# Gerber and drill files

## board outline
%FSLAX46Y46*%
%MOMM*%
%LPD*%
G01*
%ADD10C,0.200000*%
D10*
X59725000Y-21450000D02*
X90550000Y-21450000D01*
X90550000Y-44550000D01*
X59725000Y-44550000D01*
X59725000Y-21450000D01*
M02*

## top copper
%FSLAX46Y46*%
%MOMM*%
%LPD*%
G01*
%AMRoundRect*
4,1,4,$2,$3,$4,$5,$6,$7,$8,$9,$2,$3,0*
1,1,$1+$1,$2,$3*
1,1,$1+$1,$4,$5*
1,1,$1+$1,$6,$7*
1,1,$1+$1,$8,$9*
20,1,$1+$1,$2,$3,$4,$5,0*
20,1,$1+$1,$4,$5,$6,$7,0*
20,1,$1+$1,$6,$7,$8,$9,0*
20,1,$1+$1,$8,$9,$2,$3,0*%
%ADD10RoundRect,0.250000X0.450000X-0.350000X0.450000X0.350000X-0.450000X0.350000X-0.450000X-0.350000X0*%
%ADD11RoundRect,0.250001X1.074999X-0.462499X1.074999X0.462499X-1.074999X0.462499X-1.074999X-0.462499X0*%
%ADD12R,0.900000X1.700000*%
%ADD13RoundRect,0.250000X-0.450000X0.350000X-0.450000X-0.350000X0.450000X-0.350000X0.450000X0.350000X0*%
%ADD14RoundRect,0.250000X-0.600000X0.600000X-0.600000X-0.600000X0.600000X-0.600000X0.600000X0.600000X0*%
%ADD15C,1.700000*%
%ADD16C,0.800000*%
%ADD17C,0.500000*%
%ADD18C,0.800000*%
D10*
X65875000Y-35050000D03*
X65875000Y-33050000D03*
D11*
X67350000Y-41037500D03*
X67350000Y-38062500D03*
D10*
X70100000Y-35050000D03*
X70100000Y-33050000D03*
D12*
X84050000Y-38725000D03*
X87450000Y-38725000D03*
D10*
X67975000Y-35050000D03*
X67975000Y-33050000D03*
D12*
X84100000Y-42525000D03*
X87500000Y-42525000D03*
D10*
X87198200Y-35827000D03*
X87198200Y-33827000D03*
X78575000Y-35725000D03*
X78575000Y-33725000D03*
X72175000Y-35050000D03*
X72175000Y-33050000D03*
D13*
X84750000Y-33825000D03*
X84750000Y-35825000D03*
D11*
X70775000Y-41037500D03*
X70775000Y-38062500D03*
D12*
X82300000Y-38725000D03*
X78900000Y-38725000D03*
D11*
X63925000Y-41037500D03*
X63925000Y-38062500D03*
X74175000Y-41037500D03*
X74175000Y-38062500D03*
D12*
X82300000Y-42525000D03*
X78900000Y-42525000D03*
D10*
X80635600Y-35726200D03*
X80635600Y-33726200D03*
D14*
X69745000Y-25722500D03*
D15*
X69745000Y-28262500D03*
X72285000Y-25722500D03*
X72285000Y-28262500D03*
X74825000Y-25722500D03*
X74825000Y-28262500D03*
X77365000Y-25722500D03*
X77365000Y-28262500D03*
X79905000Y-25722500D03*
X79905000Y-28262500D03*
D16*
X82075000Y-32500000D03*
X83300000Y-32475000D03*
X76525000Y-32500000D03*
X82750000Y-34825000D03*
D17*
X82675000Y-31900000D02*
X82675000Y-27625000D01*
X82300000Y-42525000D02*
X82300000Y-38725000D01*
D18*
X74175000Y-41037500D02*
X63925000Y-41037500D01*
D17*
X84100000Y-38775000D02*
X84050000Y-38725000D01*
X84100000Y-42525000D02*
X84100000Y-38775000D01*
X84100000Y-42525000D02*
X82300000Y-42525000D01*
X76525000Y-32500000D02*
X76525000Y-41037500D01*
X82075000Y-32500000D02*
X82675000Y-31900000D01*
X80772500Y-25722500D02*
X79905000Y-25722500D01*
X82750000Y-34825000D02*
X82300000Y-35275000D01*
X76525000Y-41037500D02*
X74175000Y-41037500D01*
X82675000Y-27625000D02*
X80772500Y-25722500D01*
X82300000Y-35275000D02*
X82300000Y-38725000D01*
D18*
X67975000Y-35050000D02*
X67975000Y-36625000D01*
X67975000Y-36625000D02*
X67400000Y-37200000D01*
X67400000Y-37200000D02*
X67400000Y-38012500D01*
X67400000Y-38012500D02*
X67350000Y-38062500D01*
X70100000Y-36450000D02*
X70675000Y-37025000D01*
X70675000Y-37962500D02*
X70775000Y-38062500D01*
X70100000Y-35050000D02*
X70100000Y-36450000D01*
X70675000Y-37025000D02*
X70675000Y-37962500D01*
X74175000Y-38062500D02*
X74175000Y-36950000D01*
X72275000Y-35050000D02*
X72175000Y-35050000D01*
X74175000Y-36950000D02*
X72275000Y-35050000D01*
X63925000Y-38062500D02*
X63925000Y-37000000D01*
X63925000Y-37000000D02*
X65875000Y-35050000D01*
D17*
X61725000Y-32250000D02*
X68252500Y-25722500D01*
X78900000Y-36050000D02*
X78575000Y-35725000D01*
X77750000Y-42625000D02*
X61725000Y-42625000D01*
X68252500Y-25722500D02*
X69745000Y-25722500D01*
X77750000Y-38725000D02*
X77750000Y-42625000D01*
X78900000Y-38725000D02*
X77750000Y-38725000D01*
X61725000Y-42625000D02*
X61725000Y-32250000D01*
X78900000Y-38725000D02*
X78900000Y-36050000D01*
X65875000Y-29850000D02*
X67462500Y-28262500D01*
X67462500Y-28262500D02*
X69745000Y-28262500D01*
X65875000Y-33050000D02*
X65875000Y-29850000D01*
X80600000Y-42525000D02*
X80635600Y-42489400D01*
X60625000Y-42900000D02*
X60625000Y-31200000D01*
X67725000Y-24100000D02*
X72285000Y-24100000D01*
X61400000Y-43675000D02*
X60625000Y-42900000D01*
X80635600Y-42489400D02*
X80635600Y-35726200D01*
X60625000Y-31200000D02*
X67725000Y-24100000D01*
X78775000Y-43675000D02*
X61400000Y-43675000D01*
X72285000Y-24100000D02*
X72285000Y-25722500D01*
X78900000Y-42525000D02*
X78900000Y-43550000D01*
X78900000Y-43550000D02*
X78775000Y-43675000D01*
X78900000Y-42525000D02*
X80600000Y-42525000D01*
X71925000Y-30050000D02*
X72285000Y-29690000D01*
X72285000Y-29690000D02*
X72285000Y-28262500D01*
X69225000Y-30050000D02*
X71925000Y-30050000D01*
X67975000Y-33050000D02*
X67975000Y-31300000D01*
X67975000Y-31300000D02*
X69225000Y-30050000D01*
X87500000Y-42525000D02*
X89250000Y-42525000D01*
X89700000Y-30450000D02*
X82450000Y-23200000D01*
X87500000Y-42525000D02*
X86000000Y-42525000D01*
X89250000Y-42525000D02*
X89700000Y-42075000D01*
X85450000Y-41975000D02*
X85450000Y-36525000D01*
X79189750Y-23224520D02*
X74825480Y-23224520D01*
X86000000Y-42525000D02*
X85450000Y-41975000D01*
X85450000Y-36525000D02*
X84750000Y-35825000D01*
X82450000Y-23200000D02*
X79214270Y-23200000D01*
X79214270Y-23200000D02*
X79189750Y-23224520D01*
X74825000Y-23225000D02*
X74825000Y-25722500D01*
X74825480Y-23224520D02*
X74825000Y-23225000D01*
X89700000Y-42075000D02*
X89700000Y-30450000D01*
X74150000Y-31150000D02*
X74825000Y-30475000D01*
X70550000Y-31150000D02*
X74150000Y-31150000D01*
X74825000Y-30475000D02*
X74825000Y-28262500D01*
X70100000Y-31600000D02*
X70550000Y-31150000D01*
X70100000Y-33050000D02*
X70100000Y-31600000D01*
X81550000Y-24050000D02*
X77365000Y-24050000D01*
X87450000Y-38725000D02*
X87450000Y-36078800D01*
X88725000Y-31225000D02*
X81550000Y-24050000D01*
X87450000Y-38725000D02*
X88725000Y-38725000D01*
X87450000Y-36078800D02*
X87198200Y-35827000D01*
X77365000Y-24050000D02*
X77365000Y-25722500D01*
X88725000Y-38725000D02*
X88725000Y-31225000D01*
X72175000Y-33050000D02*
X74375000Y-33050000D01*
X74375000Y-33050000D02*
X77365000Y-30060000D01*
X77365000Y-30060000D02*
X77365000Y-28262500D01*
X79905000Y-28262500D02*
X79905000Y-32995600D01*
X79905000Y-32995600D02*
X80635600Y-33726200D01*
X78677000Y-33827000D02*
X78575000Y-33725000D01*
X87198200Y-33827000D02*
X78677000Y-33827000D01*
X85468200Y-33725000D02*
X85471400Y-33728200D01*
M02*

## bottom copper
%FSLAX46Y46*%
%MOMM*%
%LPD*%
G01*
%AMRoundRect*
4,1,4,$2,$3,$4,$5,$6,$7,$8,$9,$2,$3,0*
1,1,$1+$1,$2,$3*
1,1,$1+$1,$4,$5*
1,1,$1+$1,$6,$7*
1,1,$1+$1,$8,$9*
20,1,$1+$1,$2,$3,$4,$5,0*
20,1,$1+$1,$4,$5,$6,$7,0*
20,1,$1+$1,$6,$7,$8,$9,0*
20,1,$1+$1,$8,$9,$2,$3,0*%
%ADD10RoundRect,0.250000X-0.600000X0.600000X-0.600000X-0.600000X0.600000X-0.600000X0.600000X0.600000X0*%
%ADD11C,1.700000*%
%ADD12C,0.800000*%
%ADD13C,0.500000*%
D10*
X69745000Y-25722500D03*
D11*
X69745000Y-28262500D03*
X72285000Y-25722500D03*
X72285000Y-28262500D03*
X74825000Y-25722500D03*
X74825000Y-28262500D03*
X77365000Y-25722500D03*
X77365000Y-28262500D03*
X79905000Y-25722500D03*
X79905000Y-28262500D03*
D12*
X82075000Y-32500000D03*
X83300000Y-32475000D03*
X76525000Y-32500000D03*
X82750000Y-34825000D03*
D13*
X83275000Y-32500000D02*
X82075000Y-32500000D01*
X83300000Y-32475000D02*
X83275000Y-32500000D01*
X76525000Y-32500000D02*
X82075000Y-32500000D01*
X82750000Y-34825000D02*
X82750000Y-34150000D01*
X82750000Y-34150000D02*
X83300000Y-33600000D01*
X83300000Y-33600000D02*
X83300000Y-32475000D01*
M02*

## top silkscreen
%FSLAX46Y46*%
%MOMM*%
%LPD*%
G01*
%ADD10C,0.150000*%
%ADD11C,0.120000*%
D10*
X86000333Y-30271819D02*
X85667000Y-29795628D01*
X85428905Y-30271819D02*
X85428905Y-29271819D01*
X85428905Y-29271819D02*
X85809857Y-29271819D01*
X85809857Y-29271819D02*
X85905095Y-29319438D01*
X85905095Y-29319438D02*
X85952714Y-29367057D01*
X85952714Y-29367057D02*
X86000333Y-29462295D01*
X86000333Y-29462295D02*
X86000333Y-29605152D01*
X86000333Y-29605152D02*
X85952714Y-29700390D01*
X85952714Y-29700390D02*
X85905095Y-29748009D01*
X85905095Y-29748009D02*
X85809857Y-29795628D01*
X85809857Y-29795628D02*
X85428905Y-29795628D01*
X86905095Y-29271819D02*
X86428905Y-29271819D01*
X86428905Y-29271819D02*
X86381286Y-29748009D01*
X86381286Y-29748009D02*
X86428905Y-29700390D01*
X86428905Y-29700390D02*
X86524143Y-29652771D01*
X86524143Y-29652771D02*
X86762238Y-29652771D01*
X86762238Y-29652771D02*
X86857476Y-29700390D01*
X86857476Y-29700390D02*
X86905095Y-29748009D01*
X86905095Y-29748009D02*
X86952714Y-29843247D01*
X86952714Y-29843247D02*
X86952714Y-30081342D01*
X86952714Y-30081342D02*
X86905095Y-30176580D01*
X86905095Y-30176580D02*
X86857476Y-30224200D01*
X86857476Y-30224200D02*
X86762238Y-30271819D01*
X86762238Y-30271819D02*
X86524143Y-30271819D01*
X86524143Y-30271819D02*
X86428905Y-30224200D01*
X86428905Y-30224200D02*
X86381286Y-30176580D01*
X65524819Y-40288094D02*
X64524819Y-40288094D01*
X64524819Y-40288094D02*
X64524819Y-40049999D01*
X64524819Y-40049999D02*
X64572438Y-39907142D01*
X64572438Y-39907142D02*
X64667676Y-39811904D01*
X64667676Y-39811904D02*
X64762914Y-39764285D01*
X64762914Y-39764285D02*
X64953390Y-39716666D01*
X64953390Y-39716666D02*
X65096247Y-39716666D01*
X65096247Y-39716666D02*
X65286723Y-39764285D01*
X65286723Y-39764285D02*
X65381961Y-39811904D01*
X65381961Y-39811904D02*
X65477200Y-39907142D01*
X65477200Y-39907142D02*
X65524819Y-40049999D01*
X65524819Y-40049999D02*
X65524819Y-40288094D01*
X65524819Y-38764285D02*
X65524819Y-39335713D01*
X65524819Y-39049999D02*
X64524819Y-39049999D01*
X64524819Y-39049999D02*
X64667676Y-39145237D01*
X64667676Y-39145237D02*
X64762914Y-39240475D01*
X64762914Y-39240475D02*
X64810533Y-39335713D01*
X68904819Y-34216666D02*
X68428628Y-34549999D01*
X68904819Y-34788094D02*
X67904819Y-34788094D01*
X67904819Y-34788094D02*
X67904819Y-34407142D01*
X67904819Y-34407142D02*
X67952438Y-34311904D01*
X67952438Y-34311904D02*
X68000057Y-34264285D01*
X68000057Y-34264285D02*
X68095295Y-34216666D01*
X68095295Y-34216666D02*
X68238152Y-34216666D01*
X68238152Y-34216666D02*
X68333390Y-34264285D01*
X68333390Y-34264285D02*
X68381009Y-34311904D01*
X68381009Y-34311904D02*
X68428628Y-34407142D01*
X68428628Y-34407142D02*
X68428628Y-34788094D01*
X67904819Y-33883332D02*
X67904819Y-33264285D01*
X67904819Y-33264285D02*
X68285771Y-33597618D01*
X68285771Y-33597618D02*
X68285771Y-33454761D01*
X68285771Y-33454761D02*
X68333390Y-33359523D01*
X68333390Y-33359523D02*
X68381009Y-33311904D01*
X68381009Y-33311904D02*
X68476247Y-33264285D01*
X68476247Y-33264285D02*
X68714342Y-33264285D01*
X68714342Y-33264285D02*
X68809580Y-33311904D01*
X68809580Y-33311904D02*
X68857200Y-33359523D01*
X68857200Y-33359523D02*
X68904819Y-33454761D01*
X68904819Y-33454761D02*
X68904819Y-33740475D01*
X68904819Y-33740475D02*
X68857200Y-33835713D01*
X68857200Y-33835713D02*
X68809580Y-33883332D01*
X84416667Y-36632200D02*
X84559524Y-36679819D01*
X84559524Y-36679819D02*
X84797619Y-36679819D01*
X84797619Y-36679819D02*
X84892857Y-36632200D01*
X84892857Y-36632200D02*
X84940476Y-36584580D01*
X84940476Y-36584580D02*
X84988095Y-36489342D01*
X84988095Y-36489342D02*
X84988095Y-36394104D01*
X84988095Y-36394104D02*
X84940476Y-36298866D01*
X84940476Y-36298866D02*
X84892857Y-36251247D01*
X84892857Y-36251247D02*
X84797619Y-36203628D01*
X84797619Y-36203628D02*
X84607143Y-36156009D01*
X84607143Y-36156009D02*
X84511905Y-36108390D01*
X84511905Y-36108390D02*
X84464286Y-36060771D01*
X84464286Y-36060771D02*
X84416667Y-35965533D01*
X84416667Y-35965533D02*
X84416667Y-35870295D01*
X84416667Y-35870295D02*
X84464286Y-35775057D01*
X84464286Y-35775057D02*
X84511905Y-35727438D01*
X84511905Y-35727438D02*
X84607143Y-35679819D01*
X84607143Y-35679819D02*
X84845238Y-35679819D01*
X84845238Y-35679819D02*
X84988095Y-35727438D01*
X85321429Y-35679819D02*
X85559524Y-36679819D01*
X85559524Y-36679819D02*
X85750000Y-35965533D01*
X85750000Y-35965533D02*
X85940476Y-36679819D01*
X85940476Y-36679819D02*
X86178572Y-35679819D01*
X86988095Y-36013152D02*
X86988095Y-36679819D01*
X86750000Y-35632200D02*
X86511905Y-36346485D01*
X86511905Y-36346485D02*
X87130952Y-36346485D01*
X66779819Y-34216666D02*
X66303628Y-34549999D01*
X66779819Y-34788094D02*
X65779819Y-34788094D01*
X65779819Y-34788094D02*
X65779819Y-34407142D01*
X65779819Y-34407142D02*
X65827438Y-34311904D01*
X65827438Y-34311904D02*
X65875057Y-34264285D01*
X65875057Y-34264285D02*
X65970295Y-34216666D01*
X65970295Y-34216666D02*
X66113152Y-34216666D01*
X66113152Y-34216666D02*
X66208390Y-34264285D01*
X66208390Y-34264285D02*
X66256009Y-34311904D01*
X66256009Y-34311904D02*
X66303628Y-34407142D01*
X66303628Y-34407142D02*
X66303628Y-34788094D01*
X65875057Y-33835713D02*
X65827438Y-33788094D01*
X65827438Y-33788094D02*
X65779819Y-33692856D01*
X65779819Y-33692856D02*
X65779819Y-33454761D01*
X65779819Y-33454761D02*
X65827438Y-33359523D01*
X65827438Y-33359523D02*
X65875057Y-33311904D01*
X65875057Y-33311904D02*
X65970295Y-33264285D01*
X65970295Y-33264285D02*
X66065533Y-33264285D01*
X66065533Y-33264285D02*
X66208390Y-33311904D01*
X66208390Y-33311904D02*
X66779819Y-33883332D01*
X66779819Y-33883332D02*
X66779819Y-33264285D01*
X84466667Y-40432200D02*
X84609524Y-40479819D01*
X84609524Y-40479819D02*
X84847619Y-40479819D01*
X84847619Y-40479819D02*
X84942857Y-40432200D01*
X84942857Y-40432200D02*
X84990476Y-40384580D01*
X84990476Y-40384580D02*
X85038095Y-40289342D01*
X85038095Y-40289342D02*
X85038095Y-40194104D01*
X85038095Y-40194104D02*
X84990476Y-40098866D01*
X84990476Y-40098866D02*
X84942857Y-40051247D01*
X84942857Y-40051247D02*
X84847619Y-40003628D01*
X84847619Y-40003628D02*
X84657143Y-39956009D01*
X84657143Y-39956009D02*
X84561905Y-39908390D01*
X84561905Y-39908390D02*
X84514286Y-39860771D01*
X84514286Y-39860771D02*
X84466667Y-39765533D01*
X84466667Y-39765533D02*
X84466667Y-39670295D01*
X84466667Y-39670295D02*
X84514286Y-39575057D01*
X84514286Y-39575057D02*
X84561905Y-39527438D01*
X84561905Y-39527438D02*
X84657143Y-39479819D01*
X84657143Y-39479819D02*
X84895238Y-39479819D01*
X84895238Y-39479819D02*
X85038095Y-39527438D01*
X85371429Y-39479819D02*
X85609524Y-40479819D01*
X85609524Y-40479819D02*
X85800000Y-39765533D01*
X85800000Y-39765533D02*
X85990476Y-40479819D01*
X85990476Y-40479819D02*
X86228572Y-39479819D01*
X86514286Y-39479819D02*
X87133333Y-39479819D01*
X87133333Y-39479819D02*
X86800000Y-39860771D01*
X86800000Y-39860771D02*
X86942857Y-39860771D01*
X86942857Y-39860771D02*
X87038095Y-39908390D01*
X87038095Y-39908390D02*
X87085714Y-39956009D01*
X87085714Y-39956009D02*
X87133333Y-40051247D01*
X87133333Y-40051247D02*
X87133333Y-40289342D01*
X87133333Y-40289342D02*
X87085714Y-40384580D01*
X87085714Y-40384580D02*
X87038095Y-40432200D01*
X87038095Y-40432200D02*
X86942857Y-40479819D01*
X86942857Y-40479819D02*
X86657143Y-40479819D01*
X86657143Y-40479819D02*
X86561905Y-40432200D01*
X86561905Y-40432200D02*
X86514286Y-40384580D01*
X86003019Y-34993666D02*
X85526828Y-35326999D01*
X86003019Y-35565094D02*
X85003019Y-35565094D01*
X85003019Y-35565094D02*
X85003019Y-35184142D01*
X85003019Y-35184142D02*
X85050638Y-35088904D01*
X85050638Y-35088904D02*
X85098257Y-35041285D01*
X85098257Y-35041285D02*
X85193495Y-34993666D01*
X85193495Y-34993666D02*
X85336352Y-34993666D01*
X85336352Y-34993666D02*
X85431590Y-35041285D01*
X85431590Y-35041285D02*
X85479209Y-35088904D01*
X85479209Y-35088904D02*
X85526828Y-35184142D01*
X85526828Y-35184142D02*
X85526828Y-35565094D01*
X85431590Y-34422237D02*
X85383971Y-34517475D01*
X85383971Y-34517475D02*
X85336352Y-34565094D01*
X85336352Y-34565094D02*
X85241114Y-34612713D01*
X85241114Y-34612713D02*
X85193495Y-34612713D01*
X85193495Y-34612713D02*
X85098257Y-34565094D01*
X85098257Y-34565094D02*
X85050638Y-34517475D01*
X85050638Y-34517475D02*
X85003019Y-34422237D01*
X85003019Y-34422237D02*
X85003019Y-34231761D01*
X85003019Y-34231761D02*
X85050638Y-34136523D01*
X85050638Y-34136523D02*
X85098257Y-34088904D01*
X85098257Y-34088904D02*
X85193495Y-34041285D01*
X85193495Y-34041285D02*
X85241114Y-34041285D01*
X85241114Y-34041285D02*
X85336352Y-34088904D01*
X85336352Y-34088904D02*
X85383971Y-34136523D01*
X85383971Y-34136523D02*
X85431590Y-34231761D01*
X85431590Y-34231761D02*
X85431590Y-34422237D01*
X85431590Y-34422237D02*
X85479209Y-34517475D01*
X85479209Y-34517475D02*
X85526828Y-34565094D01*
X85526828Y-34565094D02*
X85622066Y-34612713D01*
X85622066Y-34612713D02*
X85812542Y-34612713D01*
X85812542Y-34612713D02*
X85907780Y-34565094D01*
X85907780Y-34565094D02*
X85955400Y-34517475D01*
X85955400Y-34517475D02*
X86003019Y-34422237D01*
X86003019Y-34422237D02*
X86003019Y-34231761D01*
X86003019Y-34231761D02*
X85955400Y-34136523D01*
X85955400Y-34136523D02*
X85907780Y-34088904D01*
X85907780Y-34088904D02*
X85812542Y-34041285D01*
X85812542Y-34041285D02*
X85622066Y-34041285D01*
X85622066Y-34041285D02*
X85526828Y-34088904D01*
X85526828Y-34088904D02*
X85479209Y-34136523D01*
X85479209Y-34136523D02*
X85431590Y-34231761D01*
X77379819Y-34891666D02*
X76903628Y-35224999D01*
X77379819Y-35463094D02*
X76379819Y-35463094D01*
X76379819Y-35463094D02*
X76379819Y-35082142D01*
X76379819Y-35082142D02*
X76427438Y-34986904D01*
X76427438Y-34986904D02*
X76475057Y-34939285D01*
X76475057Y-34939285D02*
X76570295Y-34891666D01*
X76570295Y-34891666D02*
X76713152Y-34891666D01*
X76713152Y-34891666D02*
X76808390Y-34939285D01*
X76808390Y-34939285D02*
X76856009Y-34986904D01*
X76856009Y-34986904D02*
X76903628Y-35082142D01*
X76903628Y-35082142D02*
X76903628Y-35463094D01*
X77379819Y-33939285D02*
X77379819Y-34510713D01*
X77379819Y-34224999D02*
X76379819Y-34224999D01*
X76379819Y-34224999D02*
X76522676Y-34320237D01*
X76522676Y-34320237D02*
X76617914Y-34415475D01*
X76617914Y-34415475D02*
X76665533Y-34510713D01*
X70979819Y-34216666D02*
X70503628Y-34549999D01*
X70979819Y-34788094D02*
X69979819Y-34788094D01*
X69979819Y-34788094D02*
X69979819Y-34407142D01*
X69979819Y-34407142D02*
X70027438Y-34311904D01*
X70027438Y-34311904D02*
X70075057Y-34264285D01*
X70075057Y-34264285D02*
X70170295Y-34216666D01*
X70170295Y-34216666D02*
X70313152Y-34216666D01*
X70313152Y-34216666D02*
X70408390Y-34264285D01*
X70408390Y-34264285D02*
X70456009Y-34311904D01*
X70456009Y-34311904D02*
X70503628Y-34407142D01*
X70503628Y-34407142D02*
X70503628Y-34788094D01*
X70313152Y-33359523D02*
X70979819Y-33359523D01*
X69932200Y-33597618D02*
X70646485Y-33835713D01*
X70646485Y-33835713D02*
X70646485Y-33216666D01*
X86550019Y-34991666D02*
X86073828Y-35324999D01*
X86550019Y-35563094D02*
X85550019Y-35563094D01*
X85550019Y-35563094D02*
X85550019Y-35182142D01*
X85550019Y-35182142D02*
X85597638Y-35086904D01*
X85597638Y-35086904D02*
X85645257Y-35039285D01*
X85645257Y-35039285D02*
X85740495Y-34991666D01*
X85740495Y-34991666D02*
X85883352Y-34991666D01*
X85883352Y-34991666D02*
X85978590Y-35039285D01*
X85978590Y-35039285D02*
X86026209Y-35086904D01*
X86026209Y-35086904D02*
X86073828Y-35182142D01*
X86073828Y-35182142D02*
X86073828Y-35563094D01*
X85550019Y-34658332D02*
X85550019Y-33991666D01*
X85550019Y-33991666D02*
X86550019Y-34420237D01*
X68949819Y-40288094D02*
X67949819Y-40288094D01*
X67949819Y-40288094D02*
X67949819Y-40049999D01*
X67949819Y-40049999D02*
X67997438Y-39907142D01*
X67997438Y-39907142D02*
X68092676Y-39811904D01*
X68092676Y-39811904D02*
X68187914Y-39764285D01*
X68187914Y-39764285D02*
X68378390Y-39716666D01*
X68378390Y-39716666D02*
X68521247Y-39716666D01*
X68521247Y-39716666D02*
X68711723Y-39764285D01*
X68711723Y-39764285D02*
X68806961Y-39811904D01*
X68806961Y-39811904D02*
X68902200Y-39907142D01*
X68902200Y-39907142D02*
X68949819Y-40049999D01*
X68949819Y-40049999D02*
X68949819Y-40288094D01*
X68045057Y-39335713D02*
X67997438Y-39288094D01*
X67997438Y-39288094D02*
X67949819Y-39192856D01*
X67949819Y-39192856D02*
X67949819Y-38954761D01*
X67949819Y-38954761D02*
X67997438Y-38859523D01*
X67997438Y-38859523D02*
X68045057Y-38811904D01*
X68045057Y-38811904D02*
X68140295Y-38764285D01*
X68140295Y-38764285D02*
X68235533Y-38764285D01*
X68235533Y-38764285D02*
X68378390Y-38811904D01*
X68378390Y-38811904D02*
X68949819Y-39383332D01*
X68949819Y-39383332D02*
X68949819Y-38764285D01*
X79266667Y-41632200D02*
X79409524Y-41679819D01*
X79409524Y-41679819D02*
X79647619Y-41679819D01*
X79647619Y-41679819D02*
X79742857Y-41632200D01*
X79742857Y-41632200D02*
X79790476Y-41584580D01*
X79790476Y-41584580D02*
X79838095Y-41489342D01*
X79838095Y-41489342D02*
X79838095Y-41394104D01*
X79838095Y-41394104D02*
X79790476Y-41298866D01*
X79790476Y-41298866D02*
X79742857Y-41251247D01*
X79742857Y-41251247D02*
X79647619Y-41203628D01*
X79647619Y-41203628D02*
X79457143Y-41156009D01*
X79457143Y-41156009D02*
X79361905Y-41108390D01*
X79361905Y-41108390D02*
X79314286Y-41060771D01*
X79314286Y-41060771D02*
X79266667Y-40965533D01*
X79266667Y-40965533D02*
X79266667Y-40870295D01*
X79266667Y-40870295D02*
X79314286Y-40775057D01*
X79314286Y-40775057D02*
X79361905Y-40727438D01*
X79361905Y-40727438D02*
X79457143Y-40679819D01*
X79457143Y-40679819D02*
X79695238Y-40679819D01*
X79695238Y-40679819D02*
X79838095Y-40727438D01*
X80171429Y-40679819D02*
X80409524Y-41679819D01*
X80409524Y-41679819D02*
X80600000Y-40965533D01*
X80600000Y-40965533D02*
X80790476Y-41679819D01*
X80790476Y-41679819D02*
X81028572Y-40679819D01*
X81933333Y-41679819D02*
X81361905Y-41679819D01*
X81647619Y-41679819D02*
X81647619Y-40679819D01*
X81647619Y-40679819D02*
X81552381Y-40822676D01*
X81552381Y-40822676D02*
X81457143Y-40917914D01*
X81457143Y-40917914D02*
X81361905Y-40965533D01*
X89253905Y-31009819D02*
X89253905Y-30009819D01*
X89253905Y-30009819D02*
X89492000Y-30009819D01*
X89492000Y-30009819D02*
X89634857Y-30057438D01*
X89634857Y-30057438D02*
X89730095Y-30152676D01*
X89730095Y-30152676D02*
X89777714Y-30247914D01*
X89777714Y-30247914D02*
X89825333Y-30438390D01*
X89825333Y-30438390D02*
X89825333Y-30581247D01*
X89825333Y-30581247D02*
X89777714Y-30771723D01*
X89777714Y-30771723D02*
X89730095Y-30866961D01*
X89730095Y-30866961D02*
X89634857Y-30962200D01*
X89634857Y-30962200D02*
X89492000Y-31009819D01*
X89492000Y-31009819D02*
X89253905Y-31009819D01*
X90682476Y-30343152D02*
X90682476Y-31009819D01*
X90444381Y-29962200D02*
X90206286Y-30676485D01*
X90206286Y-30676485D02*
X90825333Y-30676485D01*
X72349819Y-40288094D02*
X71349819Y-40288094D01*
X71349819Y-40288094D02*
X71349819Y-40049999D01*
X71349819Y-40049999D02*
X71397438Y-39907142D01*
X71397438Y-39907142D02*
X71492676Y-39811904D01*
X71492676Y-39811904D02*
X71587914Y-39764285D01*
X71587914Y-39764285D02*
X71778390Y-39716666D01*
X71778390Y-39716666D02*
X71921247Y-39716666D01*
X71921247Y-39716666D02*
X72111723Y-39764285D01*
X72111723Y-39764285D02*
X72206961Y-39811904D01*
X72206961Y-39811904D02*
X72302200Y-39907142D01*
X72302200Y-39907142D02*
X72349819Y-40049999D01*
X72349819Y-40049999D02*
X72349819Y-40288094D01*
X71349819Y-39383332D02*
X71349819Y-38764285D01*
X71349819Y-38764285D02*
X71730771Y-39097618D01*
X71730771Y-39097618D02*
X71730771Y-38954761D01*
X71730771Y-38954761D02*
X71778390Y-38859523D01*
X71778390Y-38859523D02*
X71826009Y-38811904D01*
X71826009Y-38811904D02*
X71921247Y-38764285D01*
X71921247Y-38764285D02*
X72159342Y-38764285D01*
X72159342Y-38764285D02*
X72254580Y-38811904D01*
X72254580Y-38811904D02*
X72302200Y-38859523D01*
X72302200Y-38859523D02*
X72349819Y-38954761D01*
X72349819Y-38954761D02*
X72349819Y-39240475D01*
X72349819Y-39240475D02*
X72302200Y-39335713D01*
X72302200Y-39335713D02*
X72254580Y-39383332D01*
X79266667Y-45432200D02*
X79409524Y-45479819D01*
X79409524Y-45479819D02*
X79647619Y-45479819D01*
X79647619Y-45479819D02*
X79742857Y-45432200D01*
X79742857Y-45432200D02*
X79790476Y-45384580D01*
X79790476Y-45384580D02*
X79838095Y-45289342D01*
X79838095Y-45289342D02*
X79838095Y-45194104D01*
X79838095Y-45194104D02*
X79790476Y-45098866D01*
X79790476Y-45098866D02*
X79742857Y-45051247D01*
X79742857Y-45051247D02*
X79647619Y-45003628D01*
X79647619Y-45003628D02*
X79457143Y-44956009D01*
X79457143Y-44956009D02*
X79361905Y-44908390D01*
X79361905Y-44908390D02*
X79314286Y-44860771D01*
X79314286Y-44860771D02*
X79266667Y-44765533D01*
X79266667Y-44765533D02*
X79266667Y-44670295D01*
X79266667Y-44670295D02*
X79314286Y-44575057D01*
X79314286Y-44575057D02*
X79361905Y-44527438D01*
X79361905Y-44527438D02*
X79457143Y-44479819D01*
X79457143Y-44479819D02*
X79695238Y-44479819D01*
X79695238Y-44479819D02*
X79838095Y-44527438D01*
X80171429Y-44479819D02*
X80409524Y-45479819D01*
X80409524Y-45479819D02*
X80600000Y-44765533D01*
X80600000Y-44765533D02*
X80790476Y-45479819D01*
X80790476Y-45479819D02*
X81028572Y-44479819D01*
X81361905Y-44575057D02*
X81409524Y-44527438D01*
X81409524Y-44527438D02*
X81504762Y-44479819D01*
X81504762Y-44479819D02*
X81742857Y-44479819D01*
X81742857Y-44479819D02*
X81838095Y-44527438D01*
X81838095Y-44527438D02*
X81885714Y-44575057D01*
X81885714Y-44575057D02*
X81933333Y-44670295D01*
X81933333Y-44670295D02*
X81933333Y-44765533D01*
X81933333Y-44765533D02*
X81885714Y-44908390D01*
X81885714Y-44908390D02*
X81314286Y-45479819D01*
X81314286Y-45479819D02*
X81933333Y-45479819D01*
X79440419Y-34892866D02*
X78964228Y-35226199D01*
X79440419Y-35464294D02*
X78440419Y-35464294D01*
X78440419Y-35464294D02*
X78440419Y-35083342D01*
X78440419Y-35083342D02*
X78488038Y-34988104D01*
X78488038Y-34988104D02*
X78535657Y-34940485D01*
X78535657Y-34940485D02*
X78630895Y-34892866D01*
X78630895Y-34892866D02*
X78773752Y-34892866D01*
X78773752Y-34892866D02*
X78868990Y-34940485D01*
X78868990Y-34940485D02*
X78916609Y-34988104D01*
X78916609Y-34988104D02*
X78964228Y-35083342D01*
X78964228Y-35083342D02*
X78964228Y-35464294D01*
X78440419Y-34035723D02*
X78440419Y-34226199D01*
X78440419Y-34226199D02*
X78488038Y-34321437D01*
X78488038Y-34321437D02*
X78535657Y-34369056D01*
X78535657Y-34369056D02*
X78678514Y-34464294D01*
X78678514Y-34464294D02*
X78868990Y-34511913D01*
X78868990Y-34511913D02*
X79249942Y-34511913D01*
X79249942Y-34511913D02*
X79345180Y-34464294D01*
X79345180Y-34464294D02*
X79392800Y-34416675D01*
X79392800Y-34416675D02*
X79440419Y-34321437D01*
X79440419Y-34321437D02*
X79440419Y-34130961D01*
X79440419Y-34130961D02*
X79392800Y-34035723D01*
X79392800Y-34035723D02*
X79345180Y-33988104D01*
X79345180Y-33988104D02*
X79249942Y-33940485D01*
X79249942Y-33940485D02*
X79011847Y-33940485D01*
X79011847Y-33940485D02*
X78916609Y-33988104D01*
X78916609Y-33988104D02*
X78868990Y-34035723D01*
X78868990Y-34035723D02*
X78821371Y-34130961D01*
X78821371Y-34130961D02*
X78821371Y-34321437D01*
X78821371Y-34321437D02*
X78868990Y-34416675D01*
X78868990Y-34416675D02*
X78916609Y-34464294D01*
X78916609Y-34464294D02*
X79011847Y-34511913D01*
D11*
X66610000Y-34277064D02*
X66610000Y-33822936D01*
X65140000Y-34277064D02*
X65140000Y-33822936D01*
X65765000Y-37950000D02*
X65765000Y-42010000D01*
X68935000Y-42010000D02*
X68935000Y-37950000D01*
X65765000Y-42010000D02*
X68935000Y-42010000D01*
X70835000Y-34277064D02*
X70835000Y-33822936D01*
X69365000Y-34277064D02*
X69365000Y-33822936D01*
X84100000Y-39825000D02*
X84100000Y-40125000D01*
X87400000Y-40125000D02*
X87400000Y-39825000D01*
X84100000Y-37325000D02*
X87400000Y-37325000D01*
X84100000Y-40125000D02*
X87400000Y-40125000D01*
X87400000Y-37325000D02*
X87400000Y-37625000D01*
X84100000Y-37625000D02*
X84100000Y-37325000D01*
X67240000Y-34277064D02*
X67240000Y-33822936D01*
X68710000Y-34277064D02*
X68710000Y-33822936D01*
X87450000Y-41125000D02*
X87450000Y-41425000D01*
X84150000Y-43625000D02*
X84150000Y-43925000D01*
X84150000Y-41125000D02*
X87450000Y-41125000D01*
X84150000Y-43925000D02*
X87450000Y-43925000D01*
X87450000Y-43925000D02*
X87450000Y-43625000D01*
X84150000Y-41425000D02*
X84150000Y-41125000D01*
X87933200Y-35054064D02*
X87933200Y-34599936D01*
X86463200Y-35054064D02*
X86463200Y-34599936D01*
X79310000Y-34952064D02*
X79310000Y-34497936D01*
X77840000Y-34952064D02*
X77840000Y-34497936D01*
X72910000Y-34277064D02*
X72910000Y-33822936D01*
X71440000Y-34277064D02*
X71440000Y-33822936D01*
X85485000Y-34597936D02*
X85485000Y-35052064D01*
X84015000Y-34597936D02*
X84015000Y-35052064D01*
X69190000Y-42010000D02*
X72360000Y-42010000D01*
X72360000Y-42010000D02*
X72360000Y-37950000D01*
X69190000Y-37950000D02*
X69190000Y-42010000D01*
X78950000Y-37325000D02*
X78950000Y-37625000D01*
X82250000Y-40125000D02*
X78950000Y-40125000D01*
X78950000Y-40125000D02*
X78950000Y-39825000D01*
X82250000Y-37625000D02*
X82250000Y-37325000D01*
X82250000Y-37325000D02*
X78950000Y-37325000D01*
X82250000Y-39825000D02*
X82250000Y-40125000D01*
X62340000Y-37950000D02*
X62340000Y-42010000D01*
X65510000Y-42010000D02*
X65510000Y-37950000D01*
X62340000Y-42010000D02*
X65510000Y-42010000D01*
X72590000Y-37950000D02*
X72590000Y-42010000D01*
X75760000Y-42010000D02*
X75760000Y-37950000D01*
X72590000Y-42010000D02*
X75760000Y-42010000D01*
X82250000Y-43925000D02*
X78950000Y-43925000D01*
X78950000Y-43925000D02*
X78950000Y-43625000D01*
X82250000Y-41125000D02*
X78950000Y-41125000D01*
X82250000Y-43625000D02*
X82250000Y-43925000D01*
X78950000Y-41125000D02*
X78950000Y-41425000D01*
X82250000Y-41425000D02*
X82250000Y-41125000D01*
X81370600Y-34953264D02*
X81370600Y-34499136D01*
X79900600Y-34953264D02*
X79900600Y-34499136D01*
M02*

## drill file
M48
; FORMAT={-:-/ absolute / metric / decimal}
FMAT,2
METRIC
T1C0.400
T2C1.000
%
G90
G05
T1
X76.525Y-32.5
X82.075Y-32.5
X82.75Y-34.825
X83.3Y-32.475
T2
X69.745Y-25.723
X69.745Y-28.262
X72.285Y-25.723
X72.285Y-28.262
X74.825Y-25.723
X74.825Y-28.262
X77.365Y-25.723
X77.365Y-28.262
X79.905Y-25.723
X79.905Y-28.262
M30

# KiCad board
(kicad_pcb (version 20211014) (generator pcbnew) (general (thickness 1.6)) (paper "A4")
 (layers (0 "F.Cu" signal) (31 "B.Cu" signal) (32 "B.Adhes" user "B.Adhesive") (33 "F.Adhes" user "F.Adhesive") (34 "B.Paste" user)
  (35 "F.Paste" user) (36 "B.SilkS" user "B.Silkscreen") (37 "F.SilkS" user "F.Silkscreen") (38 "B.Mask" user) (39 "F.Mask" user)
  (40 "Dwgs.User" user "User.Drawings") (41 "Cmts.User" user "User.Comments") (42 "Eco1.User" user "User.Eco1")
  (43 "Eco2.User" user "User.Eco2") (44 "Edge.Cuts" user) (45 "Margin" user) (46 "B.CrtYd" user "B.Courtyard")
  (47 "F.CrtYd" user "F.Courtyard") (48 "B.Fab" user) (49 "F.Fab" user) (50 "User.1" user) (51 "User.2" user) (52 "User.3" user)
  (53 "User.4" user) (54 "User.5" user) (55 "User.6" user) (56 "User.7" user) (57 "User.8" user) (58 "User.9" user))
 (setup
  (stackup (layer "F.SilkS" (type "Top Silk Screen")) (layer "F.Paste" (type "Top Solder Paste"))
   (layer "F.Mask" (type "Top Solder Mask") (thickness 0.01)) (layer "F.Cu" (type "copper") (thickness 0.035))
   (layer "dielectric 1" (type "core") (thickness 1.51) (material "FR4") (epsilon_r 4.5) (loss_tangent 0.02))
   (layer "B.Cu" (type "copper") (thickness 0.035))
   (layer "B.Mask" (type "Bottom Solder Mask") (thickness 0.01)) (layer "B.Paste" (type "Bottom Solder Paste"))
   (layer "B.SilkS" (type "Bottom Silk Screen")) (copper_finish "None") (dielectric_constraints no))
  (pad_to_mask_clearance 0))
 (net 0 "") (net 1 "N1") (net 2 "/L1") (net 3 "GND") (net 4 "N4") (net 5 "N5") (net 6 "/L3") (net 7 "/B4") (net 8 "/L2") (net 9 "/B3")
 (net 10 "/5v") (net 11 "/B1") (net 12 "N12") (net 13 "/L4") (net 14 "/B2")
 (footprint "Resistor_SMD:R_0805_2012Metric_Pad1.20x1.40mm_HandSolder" (layer "F.Cu") (at 65.875 34.05 90)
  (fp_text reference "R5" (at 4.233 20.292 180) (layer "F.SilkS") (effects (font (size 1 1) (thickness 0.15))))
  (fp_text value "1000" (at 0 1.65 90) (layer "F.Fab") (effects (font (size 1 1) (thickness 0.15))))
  (fp_line (start -0.227064 0.735) (end 0.227064 0.735) (layer "F.SilkS") (width 0.12))
  (fp_line (start -0.227064 -0.735) (end 0.227064 -0.735) (layer "F.SilkS") (width 0.12))
  (pad "1" smd roundrect (at -1 0 90) (size 1.2 1.4) (layers "F.Cu" "F.Paste" "F.Mask") (roundrect_rratio 0.208333) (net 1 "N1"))
  (pad "2" smd roundrect (at 1 0 90) (size 1.2 1.4) (layers "F.Cu" "F.Paste" "F.Mask") (roundrect_rratio 0.208333) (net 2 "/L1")))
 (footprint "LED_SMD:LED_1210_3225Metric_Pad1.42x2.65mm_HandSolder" (layer "F.Cu") (at 67.35 39.55 90)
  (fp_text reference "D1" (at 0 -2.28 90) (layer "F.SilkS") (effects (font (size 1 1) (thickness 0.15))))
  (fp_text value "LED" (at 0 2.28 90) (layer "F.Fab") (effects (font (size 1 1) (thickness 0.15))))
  (fp_line (start 1.6 -1.585) (end -2.46 -1.585) (layer "F.SilkS") (width 0.12))
  (fp_line (start -2.46 1.585) (end 1.6 1.585) (layer "F.SilkS") (width 0.12))
  (fp_line (start -2.46 -1.585) (end -2.46 1.585) (layer "F.SilkS") (width 0.12))
  (pad "1" smd roundrect (at -1.4875 0 90) (size 1.425 2.65) (layers "F.Cu" "F.Paste" "F.Mask") (roundrect_rratio 0.175439) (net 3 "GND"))
  (pad "2" smd roundrect (at 1.4875 0 90) (size 1.425 2.65) (layers "F.Cu" "F.Paste" "F.Mask") (roundrect_rratio 0.175439) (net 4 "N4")))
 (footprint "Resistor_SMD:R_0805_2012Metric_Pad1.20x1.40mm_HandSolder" (layer "F.Cu") (at 70.1 34.05 90)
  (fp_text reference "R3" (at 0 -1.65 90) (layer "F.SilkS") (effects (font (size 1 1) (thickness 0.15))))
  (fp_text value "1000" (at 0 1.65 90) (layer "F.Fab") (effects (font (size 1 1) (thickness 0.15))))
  (fp_line (start -0.227064 0.735) (end 0.227064 0.735) (layer "F.SilkS") (width 0.12))
  (fp_line (start -0.227064 -0.735) (end 0.227064 -0.735) (layer "F.SilkS") (width 0.12))
  (pad "1" smd roundrect (at -1 0 90) (size 1.2 1.4) (layers "F.Cu" "F.Paste" "F.Mask") (roundrect_rratio 0.208333) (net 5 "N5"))
  (pad "2" smd roundrect (at 1 0 90) (size 1.2 1.4) (layers "F.Cu" "F.Paste" "F.Mask") (roundrect_rratio 0.208333) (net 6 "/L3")))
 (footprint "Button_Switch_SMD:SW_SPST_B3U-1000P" (layer "F.Cu") (at 85.75 38.725)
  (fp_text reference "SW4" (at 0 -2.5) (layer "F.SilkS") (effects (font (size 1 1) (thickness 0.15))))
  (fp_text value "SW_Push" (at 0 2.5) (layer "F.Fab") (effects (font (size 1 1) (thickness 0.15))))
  (fp_line (start -1.65 1.1) (end -1.65 1.4) (layer "F.SilkS") (width 0.12))
  (fp_line (start 1.65 1.4) (end 1.65 1.1) (layer "F.SilkS") (width 0.12))
  (fp_line (start -1.65 -1.4) (end 1.65 -1.4) (layer "F.SilkS") (width 0.12))
  (fp_line (start -1.65 1.4) (end 1.65 1.4) (layer "F.SilkS") (width 0.12))
  (fp_line (start 1.65 -1.4) (end 1.65 -1.1) (layer "F.SilkS") (width 0.12))
  (fp_line (start -1.65 -1.1) (end -1.65 -1.4) (layer "F.SilkS") (width 0.12))
  (pad "1" smd rect (at -1.7 0) (size 0.9 1.7) (layers "F.Cu" "F.Paste" "F.Mask") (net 3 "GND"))
  (pad "2" smd rect (at 1.7 0) (size 0.9 1.7) (layers "F.Cu" "F.Paste" "F.Mask") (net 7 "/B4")))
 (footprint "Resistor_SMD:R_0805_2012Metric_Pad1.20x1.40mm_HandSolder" (layer "F.Cu") (at 67.975 34.05 90)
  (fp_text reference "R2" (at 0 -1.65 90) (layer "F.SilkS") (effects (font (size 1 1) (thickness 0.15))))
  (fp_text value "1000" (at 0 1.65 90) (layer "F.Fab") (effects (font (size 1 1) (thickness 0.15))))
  (fp_line (start -0.227064 -0.735) (end 0.227064 -0.735) (layer "F.SilkS") (width 0.12))
  (fp_line (start -0.227064 0.735) (end 0.227064 0.735) (layer "F.SilkS") (width 0.12))
  (pad "1" smd roundrect (at -1 0 90) (size 1.2 1.4) (layers "F.Cu" "F.Paste" "F.Mask") (roundrect_rratio 0.208333) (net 4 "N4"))
  (pad "2" smd roundrect (at 1 0 90) (size 1.2 1.4) (layers "F.Cu" "F.Paste" "F.Mask") (roundrect_rratio 0.208333) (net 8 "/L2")))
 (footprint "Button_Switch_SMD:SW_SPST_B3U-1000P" (layer "F.Cu") (at 85.8 42.525)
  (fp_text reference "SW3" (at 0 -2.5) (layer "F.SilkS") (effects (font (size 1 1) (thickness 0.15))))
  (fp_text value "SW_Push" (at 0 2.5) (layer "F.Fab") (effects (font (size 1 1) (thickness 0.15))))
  (fp_line (start 1.65 -1.4) (end 1.65 -1.1) (layer "F.SilkS") (width 0.12))
  (fp_line (start -1.65 1.1) (end -1.65 1.4) (layer "F.SilkS") (width 0.12))
  (fp_line (start -1.65 -1.4) (end 1.65 -1.4) (layer "F.SilkS") (width 0.12))
  (fp_line (start -1.65 1.4) (end 1.65 1.4) (layer "F.SilkS") (width 0.12))
  (fp_line (start 1.65 1.4) (end 1.65 1.1) (layer "F.SilkS") (width 0.12))
  (fp_line (start -1.65 -1.1) (end -1.65 -1.4) (layer "F.SilkS") (width 0.12))
  (pad "1" smd rect (at -1.7 0) (size 0.9 1.7) (layers "F.Cu" "F.Paste" "F.Mask") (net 3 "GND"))
  (pad "2" smd rect (at 1.7 0) (size 0.9 1.7) (layers "F.Cu" "F.Paste" "F.Mask") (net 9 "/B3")))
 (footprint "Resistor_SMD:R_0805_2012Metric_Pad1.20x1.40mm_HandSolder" (layer "F.Cu") (at 87.1982 34.827 90)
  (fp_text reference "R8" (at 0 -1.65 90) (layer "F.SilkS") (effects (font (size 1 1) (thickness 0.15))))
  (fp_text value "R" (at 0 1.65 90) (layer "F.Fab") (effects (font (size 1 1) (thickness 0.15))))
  (fp_line (start -0.227064 0.735) (end 0.227064 0.735) (layer "F.SilkS") (width 0.12))
  (fp_line (start -0.227064 -0.735) (end 0.227064 -0.735) (layer "F.SilkS") (width 0.12))
  (pad "1" smd roundrect (at -1 0 90) (size 1.2 1.4) (layers "F.Cu" "F.Paste" "F.Mask") (roundrect_rratio 0.208333) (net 7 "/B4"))
  (pad "2" smd roundrect (at 1 0 90) (size 1.2 1.4) (layers "F.Cu" "F.Paste" "F.Mask") (roundrect_rratio 0.208333) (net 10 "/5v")))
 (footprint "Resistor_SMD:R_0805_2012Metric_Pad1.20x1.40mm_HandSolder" (layer "F.Cu") (at 78.575 34.725 90)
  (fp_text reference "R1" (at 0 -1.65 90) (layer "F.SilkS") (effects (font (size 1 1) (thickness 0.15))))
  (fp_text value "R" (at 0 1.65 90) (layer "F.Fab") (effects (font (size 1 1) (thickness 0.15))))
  (fp_line (start -0.227064 0.735) (end 0.227064 0.735) (layer "F.SilkS") (width 0.12))
  (fp_line (start -0.227064 -0.735) (end 0.227064 -0.735) (layer "F.SilkS") (width 0.12))
  (pad "1" smd roundrect (at -1 0 90) (size 1.2 1.4) (layers "F.Cu" "F.Paste" "F.Mask") (roundrect_rratio 0.208333) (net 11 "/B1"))
  (pad "2" smd roundrect (at 1 0 90) (size 1.2 1.4) (layers "F.Cu" "F.Paste" "F.Mask") (roundrect_rratio 0.208333) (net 10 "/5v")))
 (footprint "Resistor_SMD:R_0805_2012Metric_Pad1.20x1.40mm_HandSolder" (layer "F.Cu") (at 72.175 34.05 90)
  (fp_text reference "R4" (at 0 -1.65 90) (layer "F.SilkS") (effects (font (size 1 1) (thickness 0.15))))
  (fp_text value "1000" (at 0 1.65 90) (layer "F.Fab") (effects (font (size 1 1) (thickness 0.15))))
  (fp_line (start -0.227064 0.735) (end 0.227064 0.735) (layer "F.SilkS") (width 0.12))
  (fp_line (start -0.227064 -0.735) (end 0.227064 -0.735) (layer "F.SilkS") (width 0.12))
  (pad "1" smd roundrect (at -1 0 90) (size 1.2 1.4) (layers "F.Cu" "F.Paste" "F.Mask") (roundrect_rratio 0.208333) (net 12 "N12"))
  (pad "2" smd roundrect (at 1 0 90) (size 1.2 1.4) (layers "F.Cu" "F.Paste" "F.Mask") (roundrect_rratio 0.208333) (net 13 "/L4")))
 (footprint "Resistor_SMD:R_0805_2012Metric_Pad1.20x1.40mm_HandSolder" (layer "F.Cu") (at 84.75 34.825 -90)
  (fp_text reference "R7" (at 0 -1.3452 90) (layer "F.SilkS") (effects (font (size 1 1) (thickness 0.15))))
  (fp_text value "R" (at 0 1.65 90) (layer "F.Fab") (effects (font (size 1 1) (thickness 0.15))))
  (fp_line (start -0.227064 -0.735) (end 0.227064 -0.735) (layer "F.SilkS") (width 0.12))
  (fp_line (start -0.227064 0.735) (end 0.227064 0.735) (layer "F.SilkS") (width 0.12))
  (pad "1" smd roundrect (at -1 0 270) (size 1.2 1.4) (layers "F.Cu" "F.Paste" "F.Mask") (roundrect_rratio 0.208333) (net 10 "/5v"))
  (pad "2" smd roundrect (at 1 0 270) (size 1.2 1.4) (layers "F.Cu" "F.Paste" "F.Mask") (roundrect_rratio 0.208333) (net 9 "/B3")))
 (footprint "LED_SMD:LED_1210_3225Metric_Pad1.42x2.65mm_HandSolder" (layer "F.Cu") (at 70.775 39.55 90)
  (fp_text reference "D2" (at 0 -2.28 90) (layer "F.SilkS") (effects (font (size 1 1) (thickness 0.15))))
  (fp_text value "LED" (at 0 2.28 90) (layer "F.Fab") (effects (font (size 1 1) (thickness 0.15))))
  (fp_line (start -2.46 -1.585) (end -2.46 1.585) (layer "F.SilkS") (width 0.12))
  (fp_line (start -2.46 1.585) (end 1.6 1.585) (layer "F.SilkS") (width 0.12))
  (fp_line (start 1.6 -1.585) (end -2.46 -1.585) (layer "F.SilkS") (width 0.12))
  (pad "1" smd roundrect (at -1.4875 0 90) (size 1.425 2.65) (layers "F.Cu" "F.Paste" "F.Mask") (roundrect_rratio 0.175439) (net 3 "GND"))
  (pad "2" smd roundrect (at 1.4875 0 90) (size 1.425 2.65) (layers "F.Cu" "F.Paste" "F.Mask") (roundrect_rratio 0.175439) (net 5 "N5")))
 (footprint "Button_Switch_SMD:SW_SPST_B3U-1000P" (layer "F.Cu") (at 80.6 38.725 180)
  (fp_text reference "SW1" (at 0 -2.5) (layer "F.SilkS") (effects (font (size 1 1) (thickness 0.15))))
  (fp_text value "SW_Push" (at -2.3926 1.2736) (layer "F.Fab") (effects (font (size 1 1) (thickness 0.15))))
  (fp_line (start 1.65 1.4) (end 1.65 1.1) (layer "F.SilkS") (width 0.12))
  (fp_line (start -1.65 -1.4) (end 1.65 -1.4) (layer "F.SilkS") (width 0.12))
  (fp_line (start 1.65 -1.4) (end 1.65 -1.1) (layer "F.SilkS") (width 0.12))
  (fp_line (start -1.65 1.1) (end -1.65 1.4) (layer "F.SilkS") (width 0.12))
  (fp_line (start -1.65 1.4) (end 1.65 1.4) (layer "F.SilkS") (width 0.12))
  (fp_line (start -1.65 -1.1) (end -1.65 -1.4) (layer "F.SilkS") (width 0.12))
  (pad "1" smd rect (at -1.7 0 180) (size 0.9 1.7) (layers "F.Cu" "F.Paste" "F.Mask") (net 3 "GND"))
  (pad "2" smd rect (at 1.7 0 180) (size 0.9 1.7) (layers "F.Cu" "F.Paste" "F.Mask") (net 11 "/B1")))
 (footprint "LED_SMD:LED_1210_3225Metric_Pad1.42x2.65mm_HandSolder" (layer "F.Cu") (at 63.925 39.55 90)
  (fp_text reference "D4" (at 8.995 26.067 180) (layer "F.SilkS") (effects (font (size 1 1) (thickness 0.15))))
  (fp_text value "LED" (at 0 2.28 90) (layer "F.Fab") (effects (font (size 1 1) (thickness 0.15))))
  (fp_line (start 1.6 -1.585) (end -2.46 -1.585) (layer "F.SilkS") (width 0.12))
  (fp_line (start -2.46 1.585) (end 1.6 1.585) (layer "F.SilkS") (width 0.12))
  (fp_line (start -2.46 -1.585) (end -2.46 1.585) (layer "F.SilkS") (width 0.12))
  (pad "1" smd roundrect (at -1.4875 0 90) (size 1.425 2.65) (layers "F.Cu" "F.Paste" "F.Mask") (roundrect_rratio 0.175439) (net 3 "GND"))
  (pad "2" smd roundrect (at 1.4875 0 90) (size 1.425 2.65) (layers "F.Cu" "F.Paste" "F.Mask") (roundrect_rratio 0.175439) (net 1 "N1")))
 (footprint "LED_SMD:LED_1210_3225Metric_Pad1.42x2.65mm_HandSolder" (layer "F.Cu") (at 74.175 39.55 90)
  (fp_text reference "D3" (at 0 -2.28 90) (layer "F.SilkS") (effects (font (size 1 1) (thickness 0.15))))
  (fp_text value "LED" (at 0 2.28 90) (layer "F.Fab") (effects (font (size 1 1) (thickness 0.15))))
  (fp_line (start 1.6 -1.585) (end -2.46 -1.585) (layer "F.SilkS") (width 0.12))
  (fp_line (start -2.46 1.585) (end 1.6 1.585) (layer "F.SilkS") (width 0.12))
  (fp_line (start -2.46 -1.585) (end -2.46 1.585) (layer "F.SilkS") (width 0.12))
  (pad "1" smd roundrect (at -1.4875 0 90) (size 1.425 2.65) (layers "F.Cu" "F.Paste" "F.Mask") (roundrect_rratio 0.175439) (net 3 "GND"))
  (pad "2" smd roundrect (at 1.4875 0 90) (size 1.425 2.65) (layers "F.Cu" "F.Paste" "F.Mask") (roundrect_rratio 0.175439) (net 12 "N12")))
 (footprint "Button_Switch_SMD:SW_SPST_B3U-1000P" (layer "F.Cu") (at 80.6 42.525 180)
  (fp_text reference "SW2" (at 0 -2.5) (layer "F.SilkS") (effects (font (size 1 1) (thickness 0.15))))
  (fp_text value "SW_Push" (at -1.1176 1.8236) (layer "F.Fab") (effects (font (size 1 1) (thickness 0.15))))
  (fp_line (start -1.65 -1.4) (end 1.65 -1.4) (layer "F.SilkS") (width 0.12))
  (fp_line (start 1.65 -1.4) (end 1.65 -1.1) (layer "F.SilkS") (width 0.12))
  (fp_line (start -1.65 1.4) (end 1.65 1.4) (layer "F.SilkS") (width 0.12))
  (fp_line (start -1.65 -1.1) (end -1.65 -1.4) (layer "F.SilkS") (width 0.12))
  (fp_line (start 1.65 1.4) (end 1.65 1.1) (layer "F.SilkS") (width 0.12))
  (fp_line (start -1.65 1.1) (end -1.65 1.4) (layer "F.SilkS") (width 0.12))
  (pad "1" smd rect (at -1.7 0 180) (size 0.9 1.7) (layers "F.Cu" "F.Paste" "F.Mask") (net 3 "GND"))
  (pad "2" smd rect (at 1.7 0 180) (size 0.9 1.7) (layers "F.Cu" "F.Paste" "F.Mask") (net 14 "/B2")))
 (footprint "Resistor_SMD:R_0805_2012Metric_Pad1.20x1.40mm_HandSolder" (layer "F.Cu") (at 80.6356 34.7262 90)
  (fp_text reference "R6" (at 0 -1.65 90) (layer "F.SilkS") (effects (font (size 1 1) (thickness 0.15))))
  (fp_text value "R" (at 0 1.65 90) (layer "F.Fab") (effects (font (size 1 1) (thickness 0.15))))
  (fp_line (start -0.227064 0.735) (end 0.227064 0.735) (layer "F.SilkS") (width 0.12))
  (fp_line (start -0.227064 -0.735) (end 0.227064 -0.735) (layer "F.SilkS") (width 0.12))
  (pad "1" smd roundrect (at -1 0 90) (size 1.2 1.4) (layers "F.Cu" "F.Paste" "F.Mask") (roundrect_rratio 0.208333) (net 14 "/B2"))
  (pad "2" smd roundrect (at 1 0 90) (size 1.2 1.4) (layers "F.Cu" "F.Paste" "F.Mask") (roundrect_rratio 0.208333) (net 10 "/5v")))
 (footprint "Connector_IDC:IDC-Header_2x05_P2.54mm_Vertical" (layer "B.Cu") (at 69.745 25.7225 -90)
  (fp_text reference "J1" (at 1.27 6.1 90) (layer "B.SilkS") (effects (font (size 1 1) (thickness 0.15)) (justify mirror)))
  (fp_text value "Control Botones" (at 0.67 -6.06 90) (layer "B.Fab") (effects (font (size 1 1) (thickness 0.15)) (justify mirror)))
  (pad "1" thru_hole roundrect (at 0 0 270) (size 1.7 1.7) (drill 1) (layers *.Cu *.Mask) (roundrect_rratio 0.147059) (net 11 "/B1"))
  (pad "2" thru_hole circle (at 2.54 0 270) (size 1.7 1.7) (drill 1) (layers *.Cu *.Mask) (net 2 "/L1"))
  (pad "3" thru_hole circle (at 0 -2.54 270) (size 1.7 1.7) (drill 1) (layers *.Cu *.Mask) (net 14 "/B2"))
  (pad "4" thru_hole circle (at 2.54 -2.54 270) (size 1.7 1.7) (drill 1) (layers *.Cu *.Mask) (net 8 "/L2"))
  (pad "5" thru_hole circle (at 0 -5.08 270) (size 1.7 1.7) (drill 1) (layers *.Cu *.Mask) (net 9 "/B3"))
  (pad "6" thru_hole circle (at 2.54 -5.08 270) (size 1.7 1.7) (drill 1) (layers *.Cu *.Mask) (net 6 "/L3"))
  (pad "7" thru_hole circle (at 0 -7.62 270) (size 1.7 1.7) (drill 1) (layers *.Cu *.Mask) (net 7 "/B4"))
  (pad "8" thru_hole circle (at 2.54 -7.62 270) (size 1.7 1.7) (drill 1) (layers *.Cu *.Mask) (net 13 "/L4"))
  (pad "9" thru_hole circle (at 0 -10.16 270) (size 1.7 1.7) (drill 1) (layers *.Cu *.Mask) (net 3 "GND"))
  (pad "10" thru_hole circle (at 2.54 -10.16 270) (size 1.7 1.7) (drill 1) (layers *.Cu *.Mask) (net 10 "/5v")))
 (gr_rect (start 59.725 21.45) (end 90.55 44.55) (layer "Edge.Cuts") (width 0.2) (fill none))
 (segment (start 82.675 31.9) (end 82.675 27.625) (width 0.5) (layer "F.Cu") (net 3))
 (segment (start 82.3 42.525) (end 82.3 38.725) (width 0.5) (layer "F.Cu") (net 3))
 (segment (start 74.175 41.0375) (end 63.925 41.0375) (width 0.8) (layer "F.Cu") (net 3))
 (segment (start 84.1 38.775) (end 84.05 38.725) (width 0.5) (layer "F.Cu") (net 3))
 (segment (start 84.1 42.525) (end 84.1 38.775) (width 0.5) (layer "F.Cu") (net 3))
 (segment (start 84.1 42.525) (end 82.3 42.525) (width 0.5) (layer "F.Cu") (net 3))
 (segment (start 76.525 32.5) (end 76.525 41.0375) (width 0.5) (layer "F.Cu") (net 3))
 (segment (start 82.075 32.5) (end 82.675 31.9) (width 0.5) (layer "F.Cu") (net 3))
 (segment (start 80.7725 25.7225) (end 79.905 25.7225) (width 0.5) (layer "F.Cu") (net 3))
 (segment (start 82.75 34.825) (end 82.3 35.275) (width 0.5) (layer "F.Cu") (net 3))
 (segment (start 76.525 41.0375) (end 74.175 41.0375) (width 0.5) (layer "F.Cu") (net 3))
 (segment (start 82.675 27.625) (end 80.7725 25.7225) (width 0.5) (layer "F.Cu") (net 3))
 (segment (start 82.3 35.275) (end 82.3 38.725) (width 0.5) (layer "F.Cu") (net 3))
 (via (at 82.075 32.5) (size 0.8) (drill 0.4) (layers "F.Cu" "B.Cu") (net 3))
 (via (at 83.3 32.475) (size 0.8) (drill 0.4) (layers "F.Cu" "B.Cu") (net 3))
 (via (at 76.525 32.5) (size 0.8) (drill 0.4) (layers "F.Cu" "B.Cu") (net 3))
 (via (at 82.75 34.825) (size 0.8) (drill 0.4) (layers "F.Cu" "B.Cu") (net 3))
 (segment (start 83.275 32.5) (end 82.075 32.5) (width 0.5) (layer "B.Cu") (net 3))
 (segment (start 83.3 32.475) (end 83.275 32.5) (width 0.5) (layer "B.Cu") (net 3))
 (segment (start 76.525 32.5) (end 82.075 32.5) (width 0.5) (layer "B.Cu") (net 3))
 (segment (start 82.75 34.825) (end 82.75 34.15) (width 0.5) (layer "B.Cu") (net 3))
 (segment (start 82.75 34.15) (end 83.3 33.6) (width 0.5) (layer "B.Cu") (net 3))
 (segment (start 83.3 33.6) (end 83.3 32.475) (width 0.5) (layer "B.Cu") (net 3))
 (segment (start 67.975 35.05) (end 67.975 36.625) (width 0.8) (layer "F.Cu") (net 4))
 (segment (start 67.975 36.625) (end 67.4 37.2) (width 0.8) (layer "F.Cu") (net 4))
 (segment (start 67.4 37.2) (end 67.4 38.0125) (width 0.8) (layer "F.Cu") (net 4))
 (segment (start 67.4 38.0125) (end 67.35 38.0625) (width 0.8) (layer "F.Cu") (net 4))
 (segment (start 70.1 36.45) (end 70.675 37.025) (width 0.8) (layer "F.Cu") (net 5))
 (segment (start 70.675 37.9625) (end 70.775 38.0625) (width 0.8) (layer "F.Cu") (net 5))
 (segment (start 70.1 35.05) (end 70.1 36.45) (width 0.8) (layer "F.Cu") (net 5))
 (segment (start 70.675 37.025) (end 70.675 37.9625) (width 0.8) (layer "F.Cu") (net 5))
 (segment (start 74.175 38.0625) (end 74.175 36.95) (width 0.8) (layer "F.Cu") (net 12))
 (segment (start 72.275 35.05) (end 72.175 35.05) (width 0.8) (layer "F.Cu") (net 12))
 (segment (start 74.175 36.95) (end 72.275 35.05) (width 0.8) (layer "F.Cu") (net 12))
 (segment (start 63.925 38.0625) (end 63.925 37) (width 0.8) (layer "F.Cu") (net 1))
 (segment (start 63.925 37) (end 65.875 35.05) (width 0.8) (layer "F.Cu") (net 1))
 (segment (start 61.725 32.25) (end 68.2525 25.7225) (width 0.5) (layer "F.Cu") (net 11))
 (segment (start 78.9 36.05) (end 78.575 35.725) (width 0.5) (layer "F.Cu") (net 11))
 (segment (start 77.75 42.625) (end 61.725 42.625) (width 0.5) (layer "F.Cu") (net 11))
 (segment (start 68.2525 25.7225) (end 69.745 25.7225) (width 0.5) (layer "F.Cu") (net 11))
 (segment (start 77.75 38.725) (end 77.75 42.625) (width 0.5) (layer "F.Cu") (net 11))
 (segment (start 78.9 38.725) (end 77.75 38.725) (width 0.5) (layer "F.Cu") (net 11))
 (segment (start 61.725 42.625) (end 61.725 32.25) (width 0.5) (layer "F.Cu") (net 11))
 (segment (start 78.9 38.725) (end 78.9 36.05) (width 0.5) (layer "F.Cu") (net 11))
 (segment (start 65.875 29.85) (end 67.4625 28.2625) (width 0.5) (layer "F.Cu") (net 2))
 (segment (start 67.4625 28.2625) (end 69.745 28.2625) (width 0.5) (layer "F.Cu") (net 2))
 (segment (start 65.875 33.05) (end 65.875 29.85) (width 0.5) (layer "F.Cu") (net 2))
 (segment (start 80.6 42.525) (end 80.6356 42.4894) (width 0.5) (layer "F.Cu") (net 14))
 (segment (start 60.625 42.9) (end 60.625 31.2) (width 0.5) (layer "F.Cu") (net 14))
 (segment (start 67.725 24.1) (end 72.285 24.1) (width 0.5) (layer "F.Cu") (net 14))
 (segment (start 61.4 43.675) (end 60.625 42.9) (width 0.5) (layer "F.Cu") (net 14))
 (segment (start 80.6356 42.4894) (end 80.6356 35.7262) (width 0.5) (layer "F.Cu") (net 14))
 (segment (start 60.625 31.2) (end 67.725 24.1) (width 0.5) (layer "F.Cu") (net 14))
 (segment (start 78.775 43.675) (end 61.4 43.675) (width 0.5) (layer "F.Cu") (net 14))
 (segment (start 72.285 24.1) (end 72.285 25.7225) (width 0.5) (layer "F.Cu") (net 14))
 (segment (start 78.9 42.525) (end 78.9 43.55) (width 0.5) (layer "F.Cu") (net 14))
 (segment (start 78.9 43.55) (end 78.775 43.675) (width 0.5) (layer "F.Cu") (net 14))
 (segment (start 78.9 42.525) (end 80.6 42.525) (width 0.5) (layer "F.Cu") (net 14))
 (segment (start 71.925 30.05) (end 72.285 29.69) (width 0.5) (layer "F.Cu") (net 8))
 (segment (start 72.285 29.69) (end 72.285 28.2625) (width 0.5) (layer "F.Cu") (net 8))
 (segment (start 69.225 30.05) (end 71.925 30.05) (width 0.5) (layer "F.Cu") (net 8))
 (segment (start 67.975 33.05) (end 67.975 31.3) (width 0.5) (layer "F.Cu") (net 8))
 (segment (start 67.975 31.3) (end 69.225 30.05) (width 0.5) (layer "F.Cu") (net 8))
 (segment (start 87.5 42.525) (end 89.25 42.525) (width 0.5) (layer "F.Cu") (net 9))
 (segment (start 89.7 30.45) (end 82.45 23.2) (width 0.5) (layer "F.Cu") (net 9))
 (segment (start 87.5 42.525) (end 86 42.525) (width 0.5) (layer "F.Cu") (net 9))
 (segment (start 89.25 42.525) (end 89.7 42.075) (width 0.5) (layer "F.Cu") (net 9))
 (segment (start 85.45 41.975) (end 85.45 36.525) (width 0.5) (layer "F.Cu") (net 9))
 (segment (start 79.18975 23.22452) (end 74.82548 23.22452) (width 0.5) (layer "F.Cu") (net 9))
 (segment (start 86 42.525) (end 85.45 41.975) (width 0.5) (layer "F.Cu") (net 9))
 (segment (start 85.45 36.525) (end 84.75 35.825) (width 0.5) (layer "F.Cu") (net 9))
 (segment (start 82.45 23.2) (end 79.21427 23.2) (width 0.5) (layer "F.Cu") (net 9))
 (segment (start 79.21427 23.2) (end 79.18975 23.22452) (width 0.5) (layer "F.Cu") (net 9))
 (segment (start 74.825 23.225) (end 74.825 25.7225) (width 0.5) (layer "F.Cu") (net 9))
 (segment (start 74.82548 23.22452) (end 74.825 23.225) (width 0.5) (layer "F.Cu") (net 9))
 (segment (start 89.7 42.075) (end 89.7 30.45) (width 0.5) (layer "F.Cu") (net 9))
 (segment (start 74.15 31.15) (end 74.825 30.475) (width 0.5) (layer "F.Cu") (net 6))
 (segment (start 70.55 31.15) (end 74.15 31.15) (width 0.5) (layer "F.Cu") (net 6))
 (segment (start 74.825 30.475) (end 74.825 28.2625) (width 0.5) (layer "F.Cu") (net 6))
 (segment (start 70.1 31.6) (end 70.55 31.15) (width 0.5) (layer "F.Cu") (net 6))
 (segment (start 70.1 33.05) (end 70.1 31.6) (width 0.5) (layer "F.Cu") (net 6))
 (segment (start 81.55 24.05) (end 77.365 24.05) (width 0.5) (layer "F.Cu") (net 7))
 (segment (start 87.45 38.725) (end 87.45 36.0788) (width 0.5) (layer "F.Cu") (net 7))
 (segment (start 88.725 31.225) (end 81.55 24.05) (width 0.5) (layer "F.Cu") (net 7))
 (segment (start 87.45 38.725) (end 88.725 38.725) (width 0.5) (layer "F.Cu") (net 7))
 (segment (start 87.45 36.0788) (end 87.1982 35.827) (width 0.5) (layer "F.Cu") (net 7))
 (segment (start 77.365 24.05) (end 77.365 25.7225) (width 0.5) (layer "F.Cu") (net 7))
 (segment (start 88.725 38.725) (end 88.725 31.225) (width 0.5) (layer "F.Cu") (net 7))
 (segment (start 72.175 33.05) (end 74.375 33.05) (width 0.5) (layer "F.Cu") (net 13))
 (segment (start 74.375 33.05) (end 77.365 30.06) (width 0.5) (layer "F.Cu") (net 13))
 (segment (start 77.365 30.06) (end 77.365 28.2625) (width 0.5) (layer "F.Cu") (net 13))
 (segment (start 79.905 28.2625) (end 79.905 32.9956) (width 0.5) (layer "F.Cu") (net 10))
 (segment (start 79.905 32.9956) (end 80.6356 33.7262) (width 0.5) (layer "F.Cu") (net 10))
 (segment (start 78.677 33.827) (end 78.575 33.725) (width 0.5) (layer "F.Cu") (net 10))
 (segment (start 87.1982 33.827) (end 78.677 33.827) (width 0.5) (layer "F.Cu") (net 10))
 (segment (start 85.4682 33.725) (end 85.4714 33.7282) (width 0.5) (layer "F.Cu") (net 10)))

